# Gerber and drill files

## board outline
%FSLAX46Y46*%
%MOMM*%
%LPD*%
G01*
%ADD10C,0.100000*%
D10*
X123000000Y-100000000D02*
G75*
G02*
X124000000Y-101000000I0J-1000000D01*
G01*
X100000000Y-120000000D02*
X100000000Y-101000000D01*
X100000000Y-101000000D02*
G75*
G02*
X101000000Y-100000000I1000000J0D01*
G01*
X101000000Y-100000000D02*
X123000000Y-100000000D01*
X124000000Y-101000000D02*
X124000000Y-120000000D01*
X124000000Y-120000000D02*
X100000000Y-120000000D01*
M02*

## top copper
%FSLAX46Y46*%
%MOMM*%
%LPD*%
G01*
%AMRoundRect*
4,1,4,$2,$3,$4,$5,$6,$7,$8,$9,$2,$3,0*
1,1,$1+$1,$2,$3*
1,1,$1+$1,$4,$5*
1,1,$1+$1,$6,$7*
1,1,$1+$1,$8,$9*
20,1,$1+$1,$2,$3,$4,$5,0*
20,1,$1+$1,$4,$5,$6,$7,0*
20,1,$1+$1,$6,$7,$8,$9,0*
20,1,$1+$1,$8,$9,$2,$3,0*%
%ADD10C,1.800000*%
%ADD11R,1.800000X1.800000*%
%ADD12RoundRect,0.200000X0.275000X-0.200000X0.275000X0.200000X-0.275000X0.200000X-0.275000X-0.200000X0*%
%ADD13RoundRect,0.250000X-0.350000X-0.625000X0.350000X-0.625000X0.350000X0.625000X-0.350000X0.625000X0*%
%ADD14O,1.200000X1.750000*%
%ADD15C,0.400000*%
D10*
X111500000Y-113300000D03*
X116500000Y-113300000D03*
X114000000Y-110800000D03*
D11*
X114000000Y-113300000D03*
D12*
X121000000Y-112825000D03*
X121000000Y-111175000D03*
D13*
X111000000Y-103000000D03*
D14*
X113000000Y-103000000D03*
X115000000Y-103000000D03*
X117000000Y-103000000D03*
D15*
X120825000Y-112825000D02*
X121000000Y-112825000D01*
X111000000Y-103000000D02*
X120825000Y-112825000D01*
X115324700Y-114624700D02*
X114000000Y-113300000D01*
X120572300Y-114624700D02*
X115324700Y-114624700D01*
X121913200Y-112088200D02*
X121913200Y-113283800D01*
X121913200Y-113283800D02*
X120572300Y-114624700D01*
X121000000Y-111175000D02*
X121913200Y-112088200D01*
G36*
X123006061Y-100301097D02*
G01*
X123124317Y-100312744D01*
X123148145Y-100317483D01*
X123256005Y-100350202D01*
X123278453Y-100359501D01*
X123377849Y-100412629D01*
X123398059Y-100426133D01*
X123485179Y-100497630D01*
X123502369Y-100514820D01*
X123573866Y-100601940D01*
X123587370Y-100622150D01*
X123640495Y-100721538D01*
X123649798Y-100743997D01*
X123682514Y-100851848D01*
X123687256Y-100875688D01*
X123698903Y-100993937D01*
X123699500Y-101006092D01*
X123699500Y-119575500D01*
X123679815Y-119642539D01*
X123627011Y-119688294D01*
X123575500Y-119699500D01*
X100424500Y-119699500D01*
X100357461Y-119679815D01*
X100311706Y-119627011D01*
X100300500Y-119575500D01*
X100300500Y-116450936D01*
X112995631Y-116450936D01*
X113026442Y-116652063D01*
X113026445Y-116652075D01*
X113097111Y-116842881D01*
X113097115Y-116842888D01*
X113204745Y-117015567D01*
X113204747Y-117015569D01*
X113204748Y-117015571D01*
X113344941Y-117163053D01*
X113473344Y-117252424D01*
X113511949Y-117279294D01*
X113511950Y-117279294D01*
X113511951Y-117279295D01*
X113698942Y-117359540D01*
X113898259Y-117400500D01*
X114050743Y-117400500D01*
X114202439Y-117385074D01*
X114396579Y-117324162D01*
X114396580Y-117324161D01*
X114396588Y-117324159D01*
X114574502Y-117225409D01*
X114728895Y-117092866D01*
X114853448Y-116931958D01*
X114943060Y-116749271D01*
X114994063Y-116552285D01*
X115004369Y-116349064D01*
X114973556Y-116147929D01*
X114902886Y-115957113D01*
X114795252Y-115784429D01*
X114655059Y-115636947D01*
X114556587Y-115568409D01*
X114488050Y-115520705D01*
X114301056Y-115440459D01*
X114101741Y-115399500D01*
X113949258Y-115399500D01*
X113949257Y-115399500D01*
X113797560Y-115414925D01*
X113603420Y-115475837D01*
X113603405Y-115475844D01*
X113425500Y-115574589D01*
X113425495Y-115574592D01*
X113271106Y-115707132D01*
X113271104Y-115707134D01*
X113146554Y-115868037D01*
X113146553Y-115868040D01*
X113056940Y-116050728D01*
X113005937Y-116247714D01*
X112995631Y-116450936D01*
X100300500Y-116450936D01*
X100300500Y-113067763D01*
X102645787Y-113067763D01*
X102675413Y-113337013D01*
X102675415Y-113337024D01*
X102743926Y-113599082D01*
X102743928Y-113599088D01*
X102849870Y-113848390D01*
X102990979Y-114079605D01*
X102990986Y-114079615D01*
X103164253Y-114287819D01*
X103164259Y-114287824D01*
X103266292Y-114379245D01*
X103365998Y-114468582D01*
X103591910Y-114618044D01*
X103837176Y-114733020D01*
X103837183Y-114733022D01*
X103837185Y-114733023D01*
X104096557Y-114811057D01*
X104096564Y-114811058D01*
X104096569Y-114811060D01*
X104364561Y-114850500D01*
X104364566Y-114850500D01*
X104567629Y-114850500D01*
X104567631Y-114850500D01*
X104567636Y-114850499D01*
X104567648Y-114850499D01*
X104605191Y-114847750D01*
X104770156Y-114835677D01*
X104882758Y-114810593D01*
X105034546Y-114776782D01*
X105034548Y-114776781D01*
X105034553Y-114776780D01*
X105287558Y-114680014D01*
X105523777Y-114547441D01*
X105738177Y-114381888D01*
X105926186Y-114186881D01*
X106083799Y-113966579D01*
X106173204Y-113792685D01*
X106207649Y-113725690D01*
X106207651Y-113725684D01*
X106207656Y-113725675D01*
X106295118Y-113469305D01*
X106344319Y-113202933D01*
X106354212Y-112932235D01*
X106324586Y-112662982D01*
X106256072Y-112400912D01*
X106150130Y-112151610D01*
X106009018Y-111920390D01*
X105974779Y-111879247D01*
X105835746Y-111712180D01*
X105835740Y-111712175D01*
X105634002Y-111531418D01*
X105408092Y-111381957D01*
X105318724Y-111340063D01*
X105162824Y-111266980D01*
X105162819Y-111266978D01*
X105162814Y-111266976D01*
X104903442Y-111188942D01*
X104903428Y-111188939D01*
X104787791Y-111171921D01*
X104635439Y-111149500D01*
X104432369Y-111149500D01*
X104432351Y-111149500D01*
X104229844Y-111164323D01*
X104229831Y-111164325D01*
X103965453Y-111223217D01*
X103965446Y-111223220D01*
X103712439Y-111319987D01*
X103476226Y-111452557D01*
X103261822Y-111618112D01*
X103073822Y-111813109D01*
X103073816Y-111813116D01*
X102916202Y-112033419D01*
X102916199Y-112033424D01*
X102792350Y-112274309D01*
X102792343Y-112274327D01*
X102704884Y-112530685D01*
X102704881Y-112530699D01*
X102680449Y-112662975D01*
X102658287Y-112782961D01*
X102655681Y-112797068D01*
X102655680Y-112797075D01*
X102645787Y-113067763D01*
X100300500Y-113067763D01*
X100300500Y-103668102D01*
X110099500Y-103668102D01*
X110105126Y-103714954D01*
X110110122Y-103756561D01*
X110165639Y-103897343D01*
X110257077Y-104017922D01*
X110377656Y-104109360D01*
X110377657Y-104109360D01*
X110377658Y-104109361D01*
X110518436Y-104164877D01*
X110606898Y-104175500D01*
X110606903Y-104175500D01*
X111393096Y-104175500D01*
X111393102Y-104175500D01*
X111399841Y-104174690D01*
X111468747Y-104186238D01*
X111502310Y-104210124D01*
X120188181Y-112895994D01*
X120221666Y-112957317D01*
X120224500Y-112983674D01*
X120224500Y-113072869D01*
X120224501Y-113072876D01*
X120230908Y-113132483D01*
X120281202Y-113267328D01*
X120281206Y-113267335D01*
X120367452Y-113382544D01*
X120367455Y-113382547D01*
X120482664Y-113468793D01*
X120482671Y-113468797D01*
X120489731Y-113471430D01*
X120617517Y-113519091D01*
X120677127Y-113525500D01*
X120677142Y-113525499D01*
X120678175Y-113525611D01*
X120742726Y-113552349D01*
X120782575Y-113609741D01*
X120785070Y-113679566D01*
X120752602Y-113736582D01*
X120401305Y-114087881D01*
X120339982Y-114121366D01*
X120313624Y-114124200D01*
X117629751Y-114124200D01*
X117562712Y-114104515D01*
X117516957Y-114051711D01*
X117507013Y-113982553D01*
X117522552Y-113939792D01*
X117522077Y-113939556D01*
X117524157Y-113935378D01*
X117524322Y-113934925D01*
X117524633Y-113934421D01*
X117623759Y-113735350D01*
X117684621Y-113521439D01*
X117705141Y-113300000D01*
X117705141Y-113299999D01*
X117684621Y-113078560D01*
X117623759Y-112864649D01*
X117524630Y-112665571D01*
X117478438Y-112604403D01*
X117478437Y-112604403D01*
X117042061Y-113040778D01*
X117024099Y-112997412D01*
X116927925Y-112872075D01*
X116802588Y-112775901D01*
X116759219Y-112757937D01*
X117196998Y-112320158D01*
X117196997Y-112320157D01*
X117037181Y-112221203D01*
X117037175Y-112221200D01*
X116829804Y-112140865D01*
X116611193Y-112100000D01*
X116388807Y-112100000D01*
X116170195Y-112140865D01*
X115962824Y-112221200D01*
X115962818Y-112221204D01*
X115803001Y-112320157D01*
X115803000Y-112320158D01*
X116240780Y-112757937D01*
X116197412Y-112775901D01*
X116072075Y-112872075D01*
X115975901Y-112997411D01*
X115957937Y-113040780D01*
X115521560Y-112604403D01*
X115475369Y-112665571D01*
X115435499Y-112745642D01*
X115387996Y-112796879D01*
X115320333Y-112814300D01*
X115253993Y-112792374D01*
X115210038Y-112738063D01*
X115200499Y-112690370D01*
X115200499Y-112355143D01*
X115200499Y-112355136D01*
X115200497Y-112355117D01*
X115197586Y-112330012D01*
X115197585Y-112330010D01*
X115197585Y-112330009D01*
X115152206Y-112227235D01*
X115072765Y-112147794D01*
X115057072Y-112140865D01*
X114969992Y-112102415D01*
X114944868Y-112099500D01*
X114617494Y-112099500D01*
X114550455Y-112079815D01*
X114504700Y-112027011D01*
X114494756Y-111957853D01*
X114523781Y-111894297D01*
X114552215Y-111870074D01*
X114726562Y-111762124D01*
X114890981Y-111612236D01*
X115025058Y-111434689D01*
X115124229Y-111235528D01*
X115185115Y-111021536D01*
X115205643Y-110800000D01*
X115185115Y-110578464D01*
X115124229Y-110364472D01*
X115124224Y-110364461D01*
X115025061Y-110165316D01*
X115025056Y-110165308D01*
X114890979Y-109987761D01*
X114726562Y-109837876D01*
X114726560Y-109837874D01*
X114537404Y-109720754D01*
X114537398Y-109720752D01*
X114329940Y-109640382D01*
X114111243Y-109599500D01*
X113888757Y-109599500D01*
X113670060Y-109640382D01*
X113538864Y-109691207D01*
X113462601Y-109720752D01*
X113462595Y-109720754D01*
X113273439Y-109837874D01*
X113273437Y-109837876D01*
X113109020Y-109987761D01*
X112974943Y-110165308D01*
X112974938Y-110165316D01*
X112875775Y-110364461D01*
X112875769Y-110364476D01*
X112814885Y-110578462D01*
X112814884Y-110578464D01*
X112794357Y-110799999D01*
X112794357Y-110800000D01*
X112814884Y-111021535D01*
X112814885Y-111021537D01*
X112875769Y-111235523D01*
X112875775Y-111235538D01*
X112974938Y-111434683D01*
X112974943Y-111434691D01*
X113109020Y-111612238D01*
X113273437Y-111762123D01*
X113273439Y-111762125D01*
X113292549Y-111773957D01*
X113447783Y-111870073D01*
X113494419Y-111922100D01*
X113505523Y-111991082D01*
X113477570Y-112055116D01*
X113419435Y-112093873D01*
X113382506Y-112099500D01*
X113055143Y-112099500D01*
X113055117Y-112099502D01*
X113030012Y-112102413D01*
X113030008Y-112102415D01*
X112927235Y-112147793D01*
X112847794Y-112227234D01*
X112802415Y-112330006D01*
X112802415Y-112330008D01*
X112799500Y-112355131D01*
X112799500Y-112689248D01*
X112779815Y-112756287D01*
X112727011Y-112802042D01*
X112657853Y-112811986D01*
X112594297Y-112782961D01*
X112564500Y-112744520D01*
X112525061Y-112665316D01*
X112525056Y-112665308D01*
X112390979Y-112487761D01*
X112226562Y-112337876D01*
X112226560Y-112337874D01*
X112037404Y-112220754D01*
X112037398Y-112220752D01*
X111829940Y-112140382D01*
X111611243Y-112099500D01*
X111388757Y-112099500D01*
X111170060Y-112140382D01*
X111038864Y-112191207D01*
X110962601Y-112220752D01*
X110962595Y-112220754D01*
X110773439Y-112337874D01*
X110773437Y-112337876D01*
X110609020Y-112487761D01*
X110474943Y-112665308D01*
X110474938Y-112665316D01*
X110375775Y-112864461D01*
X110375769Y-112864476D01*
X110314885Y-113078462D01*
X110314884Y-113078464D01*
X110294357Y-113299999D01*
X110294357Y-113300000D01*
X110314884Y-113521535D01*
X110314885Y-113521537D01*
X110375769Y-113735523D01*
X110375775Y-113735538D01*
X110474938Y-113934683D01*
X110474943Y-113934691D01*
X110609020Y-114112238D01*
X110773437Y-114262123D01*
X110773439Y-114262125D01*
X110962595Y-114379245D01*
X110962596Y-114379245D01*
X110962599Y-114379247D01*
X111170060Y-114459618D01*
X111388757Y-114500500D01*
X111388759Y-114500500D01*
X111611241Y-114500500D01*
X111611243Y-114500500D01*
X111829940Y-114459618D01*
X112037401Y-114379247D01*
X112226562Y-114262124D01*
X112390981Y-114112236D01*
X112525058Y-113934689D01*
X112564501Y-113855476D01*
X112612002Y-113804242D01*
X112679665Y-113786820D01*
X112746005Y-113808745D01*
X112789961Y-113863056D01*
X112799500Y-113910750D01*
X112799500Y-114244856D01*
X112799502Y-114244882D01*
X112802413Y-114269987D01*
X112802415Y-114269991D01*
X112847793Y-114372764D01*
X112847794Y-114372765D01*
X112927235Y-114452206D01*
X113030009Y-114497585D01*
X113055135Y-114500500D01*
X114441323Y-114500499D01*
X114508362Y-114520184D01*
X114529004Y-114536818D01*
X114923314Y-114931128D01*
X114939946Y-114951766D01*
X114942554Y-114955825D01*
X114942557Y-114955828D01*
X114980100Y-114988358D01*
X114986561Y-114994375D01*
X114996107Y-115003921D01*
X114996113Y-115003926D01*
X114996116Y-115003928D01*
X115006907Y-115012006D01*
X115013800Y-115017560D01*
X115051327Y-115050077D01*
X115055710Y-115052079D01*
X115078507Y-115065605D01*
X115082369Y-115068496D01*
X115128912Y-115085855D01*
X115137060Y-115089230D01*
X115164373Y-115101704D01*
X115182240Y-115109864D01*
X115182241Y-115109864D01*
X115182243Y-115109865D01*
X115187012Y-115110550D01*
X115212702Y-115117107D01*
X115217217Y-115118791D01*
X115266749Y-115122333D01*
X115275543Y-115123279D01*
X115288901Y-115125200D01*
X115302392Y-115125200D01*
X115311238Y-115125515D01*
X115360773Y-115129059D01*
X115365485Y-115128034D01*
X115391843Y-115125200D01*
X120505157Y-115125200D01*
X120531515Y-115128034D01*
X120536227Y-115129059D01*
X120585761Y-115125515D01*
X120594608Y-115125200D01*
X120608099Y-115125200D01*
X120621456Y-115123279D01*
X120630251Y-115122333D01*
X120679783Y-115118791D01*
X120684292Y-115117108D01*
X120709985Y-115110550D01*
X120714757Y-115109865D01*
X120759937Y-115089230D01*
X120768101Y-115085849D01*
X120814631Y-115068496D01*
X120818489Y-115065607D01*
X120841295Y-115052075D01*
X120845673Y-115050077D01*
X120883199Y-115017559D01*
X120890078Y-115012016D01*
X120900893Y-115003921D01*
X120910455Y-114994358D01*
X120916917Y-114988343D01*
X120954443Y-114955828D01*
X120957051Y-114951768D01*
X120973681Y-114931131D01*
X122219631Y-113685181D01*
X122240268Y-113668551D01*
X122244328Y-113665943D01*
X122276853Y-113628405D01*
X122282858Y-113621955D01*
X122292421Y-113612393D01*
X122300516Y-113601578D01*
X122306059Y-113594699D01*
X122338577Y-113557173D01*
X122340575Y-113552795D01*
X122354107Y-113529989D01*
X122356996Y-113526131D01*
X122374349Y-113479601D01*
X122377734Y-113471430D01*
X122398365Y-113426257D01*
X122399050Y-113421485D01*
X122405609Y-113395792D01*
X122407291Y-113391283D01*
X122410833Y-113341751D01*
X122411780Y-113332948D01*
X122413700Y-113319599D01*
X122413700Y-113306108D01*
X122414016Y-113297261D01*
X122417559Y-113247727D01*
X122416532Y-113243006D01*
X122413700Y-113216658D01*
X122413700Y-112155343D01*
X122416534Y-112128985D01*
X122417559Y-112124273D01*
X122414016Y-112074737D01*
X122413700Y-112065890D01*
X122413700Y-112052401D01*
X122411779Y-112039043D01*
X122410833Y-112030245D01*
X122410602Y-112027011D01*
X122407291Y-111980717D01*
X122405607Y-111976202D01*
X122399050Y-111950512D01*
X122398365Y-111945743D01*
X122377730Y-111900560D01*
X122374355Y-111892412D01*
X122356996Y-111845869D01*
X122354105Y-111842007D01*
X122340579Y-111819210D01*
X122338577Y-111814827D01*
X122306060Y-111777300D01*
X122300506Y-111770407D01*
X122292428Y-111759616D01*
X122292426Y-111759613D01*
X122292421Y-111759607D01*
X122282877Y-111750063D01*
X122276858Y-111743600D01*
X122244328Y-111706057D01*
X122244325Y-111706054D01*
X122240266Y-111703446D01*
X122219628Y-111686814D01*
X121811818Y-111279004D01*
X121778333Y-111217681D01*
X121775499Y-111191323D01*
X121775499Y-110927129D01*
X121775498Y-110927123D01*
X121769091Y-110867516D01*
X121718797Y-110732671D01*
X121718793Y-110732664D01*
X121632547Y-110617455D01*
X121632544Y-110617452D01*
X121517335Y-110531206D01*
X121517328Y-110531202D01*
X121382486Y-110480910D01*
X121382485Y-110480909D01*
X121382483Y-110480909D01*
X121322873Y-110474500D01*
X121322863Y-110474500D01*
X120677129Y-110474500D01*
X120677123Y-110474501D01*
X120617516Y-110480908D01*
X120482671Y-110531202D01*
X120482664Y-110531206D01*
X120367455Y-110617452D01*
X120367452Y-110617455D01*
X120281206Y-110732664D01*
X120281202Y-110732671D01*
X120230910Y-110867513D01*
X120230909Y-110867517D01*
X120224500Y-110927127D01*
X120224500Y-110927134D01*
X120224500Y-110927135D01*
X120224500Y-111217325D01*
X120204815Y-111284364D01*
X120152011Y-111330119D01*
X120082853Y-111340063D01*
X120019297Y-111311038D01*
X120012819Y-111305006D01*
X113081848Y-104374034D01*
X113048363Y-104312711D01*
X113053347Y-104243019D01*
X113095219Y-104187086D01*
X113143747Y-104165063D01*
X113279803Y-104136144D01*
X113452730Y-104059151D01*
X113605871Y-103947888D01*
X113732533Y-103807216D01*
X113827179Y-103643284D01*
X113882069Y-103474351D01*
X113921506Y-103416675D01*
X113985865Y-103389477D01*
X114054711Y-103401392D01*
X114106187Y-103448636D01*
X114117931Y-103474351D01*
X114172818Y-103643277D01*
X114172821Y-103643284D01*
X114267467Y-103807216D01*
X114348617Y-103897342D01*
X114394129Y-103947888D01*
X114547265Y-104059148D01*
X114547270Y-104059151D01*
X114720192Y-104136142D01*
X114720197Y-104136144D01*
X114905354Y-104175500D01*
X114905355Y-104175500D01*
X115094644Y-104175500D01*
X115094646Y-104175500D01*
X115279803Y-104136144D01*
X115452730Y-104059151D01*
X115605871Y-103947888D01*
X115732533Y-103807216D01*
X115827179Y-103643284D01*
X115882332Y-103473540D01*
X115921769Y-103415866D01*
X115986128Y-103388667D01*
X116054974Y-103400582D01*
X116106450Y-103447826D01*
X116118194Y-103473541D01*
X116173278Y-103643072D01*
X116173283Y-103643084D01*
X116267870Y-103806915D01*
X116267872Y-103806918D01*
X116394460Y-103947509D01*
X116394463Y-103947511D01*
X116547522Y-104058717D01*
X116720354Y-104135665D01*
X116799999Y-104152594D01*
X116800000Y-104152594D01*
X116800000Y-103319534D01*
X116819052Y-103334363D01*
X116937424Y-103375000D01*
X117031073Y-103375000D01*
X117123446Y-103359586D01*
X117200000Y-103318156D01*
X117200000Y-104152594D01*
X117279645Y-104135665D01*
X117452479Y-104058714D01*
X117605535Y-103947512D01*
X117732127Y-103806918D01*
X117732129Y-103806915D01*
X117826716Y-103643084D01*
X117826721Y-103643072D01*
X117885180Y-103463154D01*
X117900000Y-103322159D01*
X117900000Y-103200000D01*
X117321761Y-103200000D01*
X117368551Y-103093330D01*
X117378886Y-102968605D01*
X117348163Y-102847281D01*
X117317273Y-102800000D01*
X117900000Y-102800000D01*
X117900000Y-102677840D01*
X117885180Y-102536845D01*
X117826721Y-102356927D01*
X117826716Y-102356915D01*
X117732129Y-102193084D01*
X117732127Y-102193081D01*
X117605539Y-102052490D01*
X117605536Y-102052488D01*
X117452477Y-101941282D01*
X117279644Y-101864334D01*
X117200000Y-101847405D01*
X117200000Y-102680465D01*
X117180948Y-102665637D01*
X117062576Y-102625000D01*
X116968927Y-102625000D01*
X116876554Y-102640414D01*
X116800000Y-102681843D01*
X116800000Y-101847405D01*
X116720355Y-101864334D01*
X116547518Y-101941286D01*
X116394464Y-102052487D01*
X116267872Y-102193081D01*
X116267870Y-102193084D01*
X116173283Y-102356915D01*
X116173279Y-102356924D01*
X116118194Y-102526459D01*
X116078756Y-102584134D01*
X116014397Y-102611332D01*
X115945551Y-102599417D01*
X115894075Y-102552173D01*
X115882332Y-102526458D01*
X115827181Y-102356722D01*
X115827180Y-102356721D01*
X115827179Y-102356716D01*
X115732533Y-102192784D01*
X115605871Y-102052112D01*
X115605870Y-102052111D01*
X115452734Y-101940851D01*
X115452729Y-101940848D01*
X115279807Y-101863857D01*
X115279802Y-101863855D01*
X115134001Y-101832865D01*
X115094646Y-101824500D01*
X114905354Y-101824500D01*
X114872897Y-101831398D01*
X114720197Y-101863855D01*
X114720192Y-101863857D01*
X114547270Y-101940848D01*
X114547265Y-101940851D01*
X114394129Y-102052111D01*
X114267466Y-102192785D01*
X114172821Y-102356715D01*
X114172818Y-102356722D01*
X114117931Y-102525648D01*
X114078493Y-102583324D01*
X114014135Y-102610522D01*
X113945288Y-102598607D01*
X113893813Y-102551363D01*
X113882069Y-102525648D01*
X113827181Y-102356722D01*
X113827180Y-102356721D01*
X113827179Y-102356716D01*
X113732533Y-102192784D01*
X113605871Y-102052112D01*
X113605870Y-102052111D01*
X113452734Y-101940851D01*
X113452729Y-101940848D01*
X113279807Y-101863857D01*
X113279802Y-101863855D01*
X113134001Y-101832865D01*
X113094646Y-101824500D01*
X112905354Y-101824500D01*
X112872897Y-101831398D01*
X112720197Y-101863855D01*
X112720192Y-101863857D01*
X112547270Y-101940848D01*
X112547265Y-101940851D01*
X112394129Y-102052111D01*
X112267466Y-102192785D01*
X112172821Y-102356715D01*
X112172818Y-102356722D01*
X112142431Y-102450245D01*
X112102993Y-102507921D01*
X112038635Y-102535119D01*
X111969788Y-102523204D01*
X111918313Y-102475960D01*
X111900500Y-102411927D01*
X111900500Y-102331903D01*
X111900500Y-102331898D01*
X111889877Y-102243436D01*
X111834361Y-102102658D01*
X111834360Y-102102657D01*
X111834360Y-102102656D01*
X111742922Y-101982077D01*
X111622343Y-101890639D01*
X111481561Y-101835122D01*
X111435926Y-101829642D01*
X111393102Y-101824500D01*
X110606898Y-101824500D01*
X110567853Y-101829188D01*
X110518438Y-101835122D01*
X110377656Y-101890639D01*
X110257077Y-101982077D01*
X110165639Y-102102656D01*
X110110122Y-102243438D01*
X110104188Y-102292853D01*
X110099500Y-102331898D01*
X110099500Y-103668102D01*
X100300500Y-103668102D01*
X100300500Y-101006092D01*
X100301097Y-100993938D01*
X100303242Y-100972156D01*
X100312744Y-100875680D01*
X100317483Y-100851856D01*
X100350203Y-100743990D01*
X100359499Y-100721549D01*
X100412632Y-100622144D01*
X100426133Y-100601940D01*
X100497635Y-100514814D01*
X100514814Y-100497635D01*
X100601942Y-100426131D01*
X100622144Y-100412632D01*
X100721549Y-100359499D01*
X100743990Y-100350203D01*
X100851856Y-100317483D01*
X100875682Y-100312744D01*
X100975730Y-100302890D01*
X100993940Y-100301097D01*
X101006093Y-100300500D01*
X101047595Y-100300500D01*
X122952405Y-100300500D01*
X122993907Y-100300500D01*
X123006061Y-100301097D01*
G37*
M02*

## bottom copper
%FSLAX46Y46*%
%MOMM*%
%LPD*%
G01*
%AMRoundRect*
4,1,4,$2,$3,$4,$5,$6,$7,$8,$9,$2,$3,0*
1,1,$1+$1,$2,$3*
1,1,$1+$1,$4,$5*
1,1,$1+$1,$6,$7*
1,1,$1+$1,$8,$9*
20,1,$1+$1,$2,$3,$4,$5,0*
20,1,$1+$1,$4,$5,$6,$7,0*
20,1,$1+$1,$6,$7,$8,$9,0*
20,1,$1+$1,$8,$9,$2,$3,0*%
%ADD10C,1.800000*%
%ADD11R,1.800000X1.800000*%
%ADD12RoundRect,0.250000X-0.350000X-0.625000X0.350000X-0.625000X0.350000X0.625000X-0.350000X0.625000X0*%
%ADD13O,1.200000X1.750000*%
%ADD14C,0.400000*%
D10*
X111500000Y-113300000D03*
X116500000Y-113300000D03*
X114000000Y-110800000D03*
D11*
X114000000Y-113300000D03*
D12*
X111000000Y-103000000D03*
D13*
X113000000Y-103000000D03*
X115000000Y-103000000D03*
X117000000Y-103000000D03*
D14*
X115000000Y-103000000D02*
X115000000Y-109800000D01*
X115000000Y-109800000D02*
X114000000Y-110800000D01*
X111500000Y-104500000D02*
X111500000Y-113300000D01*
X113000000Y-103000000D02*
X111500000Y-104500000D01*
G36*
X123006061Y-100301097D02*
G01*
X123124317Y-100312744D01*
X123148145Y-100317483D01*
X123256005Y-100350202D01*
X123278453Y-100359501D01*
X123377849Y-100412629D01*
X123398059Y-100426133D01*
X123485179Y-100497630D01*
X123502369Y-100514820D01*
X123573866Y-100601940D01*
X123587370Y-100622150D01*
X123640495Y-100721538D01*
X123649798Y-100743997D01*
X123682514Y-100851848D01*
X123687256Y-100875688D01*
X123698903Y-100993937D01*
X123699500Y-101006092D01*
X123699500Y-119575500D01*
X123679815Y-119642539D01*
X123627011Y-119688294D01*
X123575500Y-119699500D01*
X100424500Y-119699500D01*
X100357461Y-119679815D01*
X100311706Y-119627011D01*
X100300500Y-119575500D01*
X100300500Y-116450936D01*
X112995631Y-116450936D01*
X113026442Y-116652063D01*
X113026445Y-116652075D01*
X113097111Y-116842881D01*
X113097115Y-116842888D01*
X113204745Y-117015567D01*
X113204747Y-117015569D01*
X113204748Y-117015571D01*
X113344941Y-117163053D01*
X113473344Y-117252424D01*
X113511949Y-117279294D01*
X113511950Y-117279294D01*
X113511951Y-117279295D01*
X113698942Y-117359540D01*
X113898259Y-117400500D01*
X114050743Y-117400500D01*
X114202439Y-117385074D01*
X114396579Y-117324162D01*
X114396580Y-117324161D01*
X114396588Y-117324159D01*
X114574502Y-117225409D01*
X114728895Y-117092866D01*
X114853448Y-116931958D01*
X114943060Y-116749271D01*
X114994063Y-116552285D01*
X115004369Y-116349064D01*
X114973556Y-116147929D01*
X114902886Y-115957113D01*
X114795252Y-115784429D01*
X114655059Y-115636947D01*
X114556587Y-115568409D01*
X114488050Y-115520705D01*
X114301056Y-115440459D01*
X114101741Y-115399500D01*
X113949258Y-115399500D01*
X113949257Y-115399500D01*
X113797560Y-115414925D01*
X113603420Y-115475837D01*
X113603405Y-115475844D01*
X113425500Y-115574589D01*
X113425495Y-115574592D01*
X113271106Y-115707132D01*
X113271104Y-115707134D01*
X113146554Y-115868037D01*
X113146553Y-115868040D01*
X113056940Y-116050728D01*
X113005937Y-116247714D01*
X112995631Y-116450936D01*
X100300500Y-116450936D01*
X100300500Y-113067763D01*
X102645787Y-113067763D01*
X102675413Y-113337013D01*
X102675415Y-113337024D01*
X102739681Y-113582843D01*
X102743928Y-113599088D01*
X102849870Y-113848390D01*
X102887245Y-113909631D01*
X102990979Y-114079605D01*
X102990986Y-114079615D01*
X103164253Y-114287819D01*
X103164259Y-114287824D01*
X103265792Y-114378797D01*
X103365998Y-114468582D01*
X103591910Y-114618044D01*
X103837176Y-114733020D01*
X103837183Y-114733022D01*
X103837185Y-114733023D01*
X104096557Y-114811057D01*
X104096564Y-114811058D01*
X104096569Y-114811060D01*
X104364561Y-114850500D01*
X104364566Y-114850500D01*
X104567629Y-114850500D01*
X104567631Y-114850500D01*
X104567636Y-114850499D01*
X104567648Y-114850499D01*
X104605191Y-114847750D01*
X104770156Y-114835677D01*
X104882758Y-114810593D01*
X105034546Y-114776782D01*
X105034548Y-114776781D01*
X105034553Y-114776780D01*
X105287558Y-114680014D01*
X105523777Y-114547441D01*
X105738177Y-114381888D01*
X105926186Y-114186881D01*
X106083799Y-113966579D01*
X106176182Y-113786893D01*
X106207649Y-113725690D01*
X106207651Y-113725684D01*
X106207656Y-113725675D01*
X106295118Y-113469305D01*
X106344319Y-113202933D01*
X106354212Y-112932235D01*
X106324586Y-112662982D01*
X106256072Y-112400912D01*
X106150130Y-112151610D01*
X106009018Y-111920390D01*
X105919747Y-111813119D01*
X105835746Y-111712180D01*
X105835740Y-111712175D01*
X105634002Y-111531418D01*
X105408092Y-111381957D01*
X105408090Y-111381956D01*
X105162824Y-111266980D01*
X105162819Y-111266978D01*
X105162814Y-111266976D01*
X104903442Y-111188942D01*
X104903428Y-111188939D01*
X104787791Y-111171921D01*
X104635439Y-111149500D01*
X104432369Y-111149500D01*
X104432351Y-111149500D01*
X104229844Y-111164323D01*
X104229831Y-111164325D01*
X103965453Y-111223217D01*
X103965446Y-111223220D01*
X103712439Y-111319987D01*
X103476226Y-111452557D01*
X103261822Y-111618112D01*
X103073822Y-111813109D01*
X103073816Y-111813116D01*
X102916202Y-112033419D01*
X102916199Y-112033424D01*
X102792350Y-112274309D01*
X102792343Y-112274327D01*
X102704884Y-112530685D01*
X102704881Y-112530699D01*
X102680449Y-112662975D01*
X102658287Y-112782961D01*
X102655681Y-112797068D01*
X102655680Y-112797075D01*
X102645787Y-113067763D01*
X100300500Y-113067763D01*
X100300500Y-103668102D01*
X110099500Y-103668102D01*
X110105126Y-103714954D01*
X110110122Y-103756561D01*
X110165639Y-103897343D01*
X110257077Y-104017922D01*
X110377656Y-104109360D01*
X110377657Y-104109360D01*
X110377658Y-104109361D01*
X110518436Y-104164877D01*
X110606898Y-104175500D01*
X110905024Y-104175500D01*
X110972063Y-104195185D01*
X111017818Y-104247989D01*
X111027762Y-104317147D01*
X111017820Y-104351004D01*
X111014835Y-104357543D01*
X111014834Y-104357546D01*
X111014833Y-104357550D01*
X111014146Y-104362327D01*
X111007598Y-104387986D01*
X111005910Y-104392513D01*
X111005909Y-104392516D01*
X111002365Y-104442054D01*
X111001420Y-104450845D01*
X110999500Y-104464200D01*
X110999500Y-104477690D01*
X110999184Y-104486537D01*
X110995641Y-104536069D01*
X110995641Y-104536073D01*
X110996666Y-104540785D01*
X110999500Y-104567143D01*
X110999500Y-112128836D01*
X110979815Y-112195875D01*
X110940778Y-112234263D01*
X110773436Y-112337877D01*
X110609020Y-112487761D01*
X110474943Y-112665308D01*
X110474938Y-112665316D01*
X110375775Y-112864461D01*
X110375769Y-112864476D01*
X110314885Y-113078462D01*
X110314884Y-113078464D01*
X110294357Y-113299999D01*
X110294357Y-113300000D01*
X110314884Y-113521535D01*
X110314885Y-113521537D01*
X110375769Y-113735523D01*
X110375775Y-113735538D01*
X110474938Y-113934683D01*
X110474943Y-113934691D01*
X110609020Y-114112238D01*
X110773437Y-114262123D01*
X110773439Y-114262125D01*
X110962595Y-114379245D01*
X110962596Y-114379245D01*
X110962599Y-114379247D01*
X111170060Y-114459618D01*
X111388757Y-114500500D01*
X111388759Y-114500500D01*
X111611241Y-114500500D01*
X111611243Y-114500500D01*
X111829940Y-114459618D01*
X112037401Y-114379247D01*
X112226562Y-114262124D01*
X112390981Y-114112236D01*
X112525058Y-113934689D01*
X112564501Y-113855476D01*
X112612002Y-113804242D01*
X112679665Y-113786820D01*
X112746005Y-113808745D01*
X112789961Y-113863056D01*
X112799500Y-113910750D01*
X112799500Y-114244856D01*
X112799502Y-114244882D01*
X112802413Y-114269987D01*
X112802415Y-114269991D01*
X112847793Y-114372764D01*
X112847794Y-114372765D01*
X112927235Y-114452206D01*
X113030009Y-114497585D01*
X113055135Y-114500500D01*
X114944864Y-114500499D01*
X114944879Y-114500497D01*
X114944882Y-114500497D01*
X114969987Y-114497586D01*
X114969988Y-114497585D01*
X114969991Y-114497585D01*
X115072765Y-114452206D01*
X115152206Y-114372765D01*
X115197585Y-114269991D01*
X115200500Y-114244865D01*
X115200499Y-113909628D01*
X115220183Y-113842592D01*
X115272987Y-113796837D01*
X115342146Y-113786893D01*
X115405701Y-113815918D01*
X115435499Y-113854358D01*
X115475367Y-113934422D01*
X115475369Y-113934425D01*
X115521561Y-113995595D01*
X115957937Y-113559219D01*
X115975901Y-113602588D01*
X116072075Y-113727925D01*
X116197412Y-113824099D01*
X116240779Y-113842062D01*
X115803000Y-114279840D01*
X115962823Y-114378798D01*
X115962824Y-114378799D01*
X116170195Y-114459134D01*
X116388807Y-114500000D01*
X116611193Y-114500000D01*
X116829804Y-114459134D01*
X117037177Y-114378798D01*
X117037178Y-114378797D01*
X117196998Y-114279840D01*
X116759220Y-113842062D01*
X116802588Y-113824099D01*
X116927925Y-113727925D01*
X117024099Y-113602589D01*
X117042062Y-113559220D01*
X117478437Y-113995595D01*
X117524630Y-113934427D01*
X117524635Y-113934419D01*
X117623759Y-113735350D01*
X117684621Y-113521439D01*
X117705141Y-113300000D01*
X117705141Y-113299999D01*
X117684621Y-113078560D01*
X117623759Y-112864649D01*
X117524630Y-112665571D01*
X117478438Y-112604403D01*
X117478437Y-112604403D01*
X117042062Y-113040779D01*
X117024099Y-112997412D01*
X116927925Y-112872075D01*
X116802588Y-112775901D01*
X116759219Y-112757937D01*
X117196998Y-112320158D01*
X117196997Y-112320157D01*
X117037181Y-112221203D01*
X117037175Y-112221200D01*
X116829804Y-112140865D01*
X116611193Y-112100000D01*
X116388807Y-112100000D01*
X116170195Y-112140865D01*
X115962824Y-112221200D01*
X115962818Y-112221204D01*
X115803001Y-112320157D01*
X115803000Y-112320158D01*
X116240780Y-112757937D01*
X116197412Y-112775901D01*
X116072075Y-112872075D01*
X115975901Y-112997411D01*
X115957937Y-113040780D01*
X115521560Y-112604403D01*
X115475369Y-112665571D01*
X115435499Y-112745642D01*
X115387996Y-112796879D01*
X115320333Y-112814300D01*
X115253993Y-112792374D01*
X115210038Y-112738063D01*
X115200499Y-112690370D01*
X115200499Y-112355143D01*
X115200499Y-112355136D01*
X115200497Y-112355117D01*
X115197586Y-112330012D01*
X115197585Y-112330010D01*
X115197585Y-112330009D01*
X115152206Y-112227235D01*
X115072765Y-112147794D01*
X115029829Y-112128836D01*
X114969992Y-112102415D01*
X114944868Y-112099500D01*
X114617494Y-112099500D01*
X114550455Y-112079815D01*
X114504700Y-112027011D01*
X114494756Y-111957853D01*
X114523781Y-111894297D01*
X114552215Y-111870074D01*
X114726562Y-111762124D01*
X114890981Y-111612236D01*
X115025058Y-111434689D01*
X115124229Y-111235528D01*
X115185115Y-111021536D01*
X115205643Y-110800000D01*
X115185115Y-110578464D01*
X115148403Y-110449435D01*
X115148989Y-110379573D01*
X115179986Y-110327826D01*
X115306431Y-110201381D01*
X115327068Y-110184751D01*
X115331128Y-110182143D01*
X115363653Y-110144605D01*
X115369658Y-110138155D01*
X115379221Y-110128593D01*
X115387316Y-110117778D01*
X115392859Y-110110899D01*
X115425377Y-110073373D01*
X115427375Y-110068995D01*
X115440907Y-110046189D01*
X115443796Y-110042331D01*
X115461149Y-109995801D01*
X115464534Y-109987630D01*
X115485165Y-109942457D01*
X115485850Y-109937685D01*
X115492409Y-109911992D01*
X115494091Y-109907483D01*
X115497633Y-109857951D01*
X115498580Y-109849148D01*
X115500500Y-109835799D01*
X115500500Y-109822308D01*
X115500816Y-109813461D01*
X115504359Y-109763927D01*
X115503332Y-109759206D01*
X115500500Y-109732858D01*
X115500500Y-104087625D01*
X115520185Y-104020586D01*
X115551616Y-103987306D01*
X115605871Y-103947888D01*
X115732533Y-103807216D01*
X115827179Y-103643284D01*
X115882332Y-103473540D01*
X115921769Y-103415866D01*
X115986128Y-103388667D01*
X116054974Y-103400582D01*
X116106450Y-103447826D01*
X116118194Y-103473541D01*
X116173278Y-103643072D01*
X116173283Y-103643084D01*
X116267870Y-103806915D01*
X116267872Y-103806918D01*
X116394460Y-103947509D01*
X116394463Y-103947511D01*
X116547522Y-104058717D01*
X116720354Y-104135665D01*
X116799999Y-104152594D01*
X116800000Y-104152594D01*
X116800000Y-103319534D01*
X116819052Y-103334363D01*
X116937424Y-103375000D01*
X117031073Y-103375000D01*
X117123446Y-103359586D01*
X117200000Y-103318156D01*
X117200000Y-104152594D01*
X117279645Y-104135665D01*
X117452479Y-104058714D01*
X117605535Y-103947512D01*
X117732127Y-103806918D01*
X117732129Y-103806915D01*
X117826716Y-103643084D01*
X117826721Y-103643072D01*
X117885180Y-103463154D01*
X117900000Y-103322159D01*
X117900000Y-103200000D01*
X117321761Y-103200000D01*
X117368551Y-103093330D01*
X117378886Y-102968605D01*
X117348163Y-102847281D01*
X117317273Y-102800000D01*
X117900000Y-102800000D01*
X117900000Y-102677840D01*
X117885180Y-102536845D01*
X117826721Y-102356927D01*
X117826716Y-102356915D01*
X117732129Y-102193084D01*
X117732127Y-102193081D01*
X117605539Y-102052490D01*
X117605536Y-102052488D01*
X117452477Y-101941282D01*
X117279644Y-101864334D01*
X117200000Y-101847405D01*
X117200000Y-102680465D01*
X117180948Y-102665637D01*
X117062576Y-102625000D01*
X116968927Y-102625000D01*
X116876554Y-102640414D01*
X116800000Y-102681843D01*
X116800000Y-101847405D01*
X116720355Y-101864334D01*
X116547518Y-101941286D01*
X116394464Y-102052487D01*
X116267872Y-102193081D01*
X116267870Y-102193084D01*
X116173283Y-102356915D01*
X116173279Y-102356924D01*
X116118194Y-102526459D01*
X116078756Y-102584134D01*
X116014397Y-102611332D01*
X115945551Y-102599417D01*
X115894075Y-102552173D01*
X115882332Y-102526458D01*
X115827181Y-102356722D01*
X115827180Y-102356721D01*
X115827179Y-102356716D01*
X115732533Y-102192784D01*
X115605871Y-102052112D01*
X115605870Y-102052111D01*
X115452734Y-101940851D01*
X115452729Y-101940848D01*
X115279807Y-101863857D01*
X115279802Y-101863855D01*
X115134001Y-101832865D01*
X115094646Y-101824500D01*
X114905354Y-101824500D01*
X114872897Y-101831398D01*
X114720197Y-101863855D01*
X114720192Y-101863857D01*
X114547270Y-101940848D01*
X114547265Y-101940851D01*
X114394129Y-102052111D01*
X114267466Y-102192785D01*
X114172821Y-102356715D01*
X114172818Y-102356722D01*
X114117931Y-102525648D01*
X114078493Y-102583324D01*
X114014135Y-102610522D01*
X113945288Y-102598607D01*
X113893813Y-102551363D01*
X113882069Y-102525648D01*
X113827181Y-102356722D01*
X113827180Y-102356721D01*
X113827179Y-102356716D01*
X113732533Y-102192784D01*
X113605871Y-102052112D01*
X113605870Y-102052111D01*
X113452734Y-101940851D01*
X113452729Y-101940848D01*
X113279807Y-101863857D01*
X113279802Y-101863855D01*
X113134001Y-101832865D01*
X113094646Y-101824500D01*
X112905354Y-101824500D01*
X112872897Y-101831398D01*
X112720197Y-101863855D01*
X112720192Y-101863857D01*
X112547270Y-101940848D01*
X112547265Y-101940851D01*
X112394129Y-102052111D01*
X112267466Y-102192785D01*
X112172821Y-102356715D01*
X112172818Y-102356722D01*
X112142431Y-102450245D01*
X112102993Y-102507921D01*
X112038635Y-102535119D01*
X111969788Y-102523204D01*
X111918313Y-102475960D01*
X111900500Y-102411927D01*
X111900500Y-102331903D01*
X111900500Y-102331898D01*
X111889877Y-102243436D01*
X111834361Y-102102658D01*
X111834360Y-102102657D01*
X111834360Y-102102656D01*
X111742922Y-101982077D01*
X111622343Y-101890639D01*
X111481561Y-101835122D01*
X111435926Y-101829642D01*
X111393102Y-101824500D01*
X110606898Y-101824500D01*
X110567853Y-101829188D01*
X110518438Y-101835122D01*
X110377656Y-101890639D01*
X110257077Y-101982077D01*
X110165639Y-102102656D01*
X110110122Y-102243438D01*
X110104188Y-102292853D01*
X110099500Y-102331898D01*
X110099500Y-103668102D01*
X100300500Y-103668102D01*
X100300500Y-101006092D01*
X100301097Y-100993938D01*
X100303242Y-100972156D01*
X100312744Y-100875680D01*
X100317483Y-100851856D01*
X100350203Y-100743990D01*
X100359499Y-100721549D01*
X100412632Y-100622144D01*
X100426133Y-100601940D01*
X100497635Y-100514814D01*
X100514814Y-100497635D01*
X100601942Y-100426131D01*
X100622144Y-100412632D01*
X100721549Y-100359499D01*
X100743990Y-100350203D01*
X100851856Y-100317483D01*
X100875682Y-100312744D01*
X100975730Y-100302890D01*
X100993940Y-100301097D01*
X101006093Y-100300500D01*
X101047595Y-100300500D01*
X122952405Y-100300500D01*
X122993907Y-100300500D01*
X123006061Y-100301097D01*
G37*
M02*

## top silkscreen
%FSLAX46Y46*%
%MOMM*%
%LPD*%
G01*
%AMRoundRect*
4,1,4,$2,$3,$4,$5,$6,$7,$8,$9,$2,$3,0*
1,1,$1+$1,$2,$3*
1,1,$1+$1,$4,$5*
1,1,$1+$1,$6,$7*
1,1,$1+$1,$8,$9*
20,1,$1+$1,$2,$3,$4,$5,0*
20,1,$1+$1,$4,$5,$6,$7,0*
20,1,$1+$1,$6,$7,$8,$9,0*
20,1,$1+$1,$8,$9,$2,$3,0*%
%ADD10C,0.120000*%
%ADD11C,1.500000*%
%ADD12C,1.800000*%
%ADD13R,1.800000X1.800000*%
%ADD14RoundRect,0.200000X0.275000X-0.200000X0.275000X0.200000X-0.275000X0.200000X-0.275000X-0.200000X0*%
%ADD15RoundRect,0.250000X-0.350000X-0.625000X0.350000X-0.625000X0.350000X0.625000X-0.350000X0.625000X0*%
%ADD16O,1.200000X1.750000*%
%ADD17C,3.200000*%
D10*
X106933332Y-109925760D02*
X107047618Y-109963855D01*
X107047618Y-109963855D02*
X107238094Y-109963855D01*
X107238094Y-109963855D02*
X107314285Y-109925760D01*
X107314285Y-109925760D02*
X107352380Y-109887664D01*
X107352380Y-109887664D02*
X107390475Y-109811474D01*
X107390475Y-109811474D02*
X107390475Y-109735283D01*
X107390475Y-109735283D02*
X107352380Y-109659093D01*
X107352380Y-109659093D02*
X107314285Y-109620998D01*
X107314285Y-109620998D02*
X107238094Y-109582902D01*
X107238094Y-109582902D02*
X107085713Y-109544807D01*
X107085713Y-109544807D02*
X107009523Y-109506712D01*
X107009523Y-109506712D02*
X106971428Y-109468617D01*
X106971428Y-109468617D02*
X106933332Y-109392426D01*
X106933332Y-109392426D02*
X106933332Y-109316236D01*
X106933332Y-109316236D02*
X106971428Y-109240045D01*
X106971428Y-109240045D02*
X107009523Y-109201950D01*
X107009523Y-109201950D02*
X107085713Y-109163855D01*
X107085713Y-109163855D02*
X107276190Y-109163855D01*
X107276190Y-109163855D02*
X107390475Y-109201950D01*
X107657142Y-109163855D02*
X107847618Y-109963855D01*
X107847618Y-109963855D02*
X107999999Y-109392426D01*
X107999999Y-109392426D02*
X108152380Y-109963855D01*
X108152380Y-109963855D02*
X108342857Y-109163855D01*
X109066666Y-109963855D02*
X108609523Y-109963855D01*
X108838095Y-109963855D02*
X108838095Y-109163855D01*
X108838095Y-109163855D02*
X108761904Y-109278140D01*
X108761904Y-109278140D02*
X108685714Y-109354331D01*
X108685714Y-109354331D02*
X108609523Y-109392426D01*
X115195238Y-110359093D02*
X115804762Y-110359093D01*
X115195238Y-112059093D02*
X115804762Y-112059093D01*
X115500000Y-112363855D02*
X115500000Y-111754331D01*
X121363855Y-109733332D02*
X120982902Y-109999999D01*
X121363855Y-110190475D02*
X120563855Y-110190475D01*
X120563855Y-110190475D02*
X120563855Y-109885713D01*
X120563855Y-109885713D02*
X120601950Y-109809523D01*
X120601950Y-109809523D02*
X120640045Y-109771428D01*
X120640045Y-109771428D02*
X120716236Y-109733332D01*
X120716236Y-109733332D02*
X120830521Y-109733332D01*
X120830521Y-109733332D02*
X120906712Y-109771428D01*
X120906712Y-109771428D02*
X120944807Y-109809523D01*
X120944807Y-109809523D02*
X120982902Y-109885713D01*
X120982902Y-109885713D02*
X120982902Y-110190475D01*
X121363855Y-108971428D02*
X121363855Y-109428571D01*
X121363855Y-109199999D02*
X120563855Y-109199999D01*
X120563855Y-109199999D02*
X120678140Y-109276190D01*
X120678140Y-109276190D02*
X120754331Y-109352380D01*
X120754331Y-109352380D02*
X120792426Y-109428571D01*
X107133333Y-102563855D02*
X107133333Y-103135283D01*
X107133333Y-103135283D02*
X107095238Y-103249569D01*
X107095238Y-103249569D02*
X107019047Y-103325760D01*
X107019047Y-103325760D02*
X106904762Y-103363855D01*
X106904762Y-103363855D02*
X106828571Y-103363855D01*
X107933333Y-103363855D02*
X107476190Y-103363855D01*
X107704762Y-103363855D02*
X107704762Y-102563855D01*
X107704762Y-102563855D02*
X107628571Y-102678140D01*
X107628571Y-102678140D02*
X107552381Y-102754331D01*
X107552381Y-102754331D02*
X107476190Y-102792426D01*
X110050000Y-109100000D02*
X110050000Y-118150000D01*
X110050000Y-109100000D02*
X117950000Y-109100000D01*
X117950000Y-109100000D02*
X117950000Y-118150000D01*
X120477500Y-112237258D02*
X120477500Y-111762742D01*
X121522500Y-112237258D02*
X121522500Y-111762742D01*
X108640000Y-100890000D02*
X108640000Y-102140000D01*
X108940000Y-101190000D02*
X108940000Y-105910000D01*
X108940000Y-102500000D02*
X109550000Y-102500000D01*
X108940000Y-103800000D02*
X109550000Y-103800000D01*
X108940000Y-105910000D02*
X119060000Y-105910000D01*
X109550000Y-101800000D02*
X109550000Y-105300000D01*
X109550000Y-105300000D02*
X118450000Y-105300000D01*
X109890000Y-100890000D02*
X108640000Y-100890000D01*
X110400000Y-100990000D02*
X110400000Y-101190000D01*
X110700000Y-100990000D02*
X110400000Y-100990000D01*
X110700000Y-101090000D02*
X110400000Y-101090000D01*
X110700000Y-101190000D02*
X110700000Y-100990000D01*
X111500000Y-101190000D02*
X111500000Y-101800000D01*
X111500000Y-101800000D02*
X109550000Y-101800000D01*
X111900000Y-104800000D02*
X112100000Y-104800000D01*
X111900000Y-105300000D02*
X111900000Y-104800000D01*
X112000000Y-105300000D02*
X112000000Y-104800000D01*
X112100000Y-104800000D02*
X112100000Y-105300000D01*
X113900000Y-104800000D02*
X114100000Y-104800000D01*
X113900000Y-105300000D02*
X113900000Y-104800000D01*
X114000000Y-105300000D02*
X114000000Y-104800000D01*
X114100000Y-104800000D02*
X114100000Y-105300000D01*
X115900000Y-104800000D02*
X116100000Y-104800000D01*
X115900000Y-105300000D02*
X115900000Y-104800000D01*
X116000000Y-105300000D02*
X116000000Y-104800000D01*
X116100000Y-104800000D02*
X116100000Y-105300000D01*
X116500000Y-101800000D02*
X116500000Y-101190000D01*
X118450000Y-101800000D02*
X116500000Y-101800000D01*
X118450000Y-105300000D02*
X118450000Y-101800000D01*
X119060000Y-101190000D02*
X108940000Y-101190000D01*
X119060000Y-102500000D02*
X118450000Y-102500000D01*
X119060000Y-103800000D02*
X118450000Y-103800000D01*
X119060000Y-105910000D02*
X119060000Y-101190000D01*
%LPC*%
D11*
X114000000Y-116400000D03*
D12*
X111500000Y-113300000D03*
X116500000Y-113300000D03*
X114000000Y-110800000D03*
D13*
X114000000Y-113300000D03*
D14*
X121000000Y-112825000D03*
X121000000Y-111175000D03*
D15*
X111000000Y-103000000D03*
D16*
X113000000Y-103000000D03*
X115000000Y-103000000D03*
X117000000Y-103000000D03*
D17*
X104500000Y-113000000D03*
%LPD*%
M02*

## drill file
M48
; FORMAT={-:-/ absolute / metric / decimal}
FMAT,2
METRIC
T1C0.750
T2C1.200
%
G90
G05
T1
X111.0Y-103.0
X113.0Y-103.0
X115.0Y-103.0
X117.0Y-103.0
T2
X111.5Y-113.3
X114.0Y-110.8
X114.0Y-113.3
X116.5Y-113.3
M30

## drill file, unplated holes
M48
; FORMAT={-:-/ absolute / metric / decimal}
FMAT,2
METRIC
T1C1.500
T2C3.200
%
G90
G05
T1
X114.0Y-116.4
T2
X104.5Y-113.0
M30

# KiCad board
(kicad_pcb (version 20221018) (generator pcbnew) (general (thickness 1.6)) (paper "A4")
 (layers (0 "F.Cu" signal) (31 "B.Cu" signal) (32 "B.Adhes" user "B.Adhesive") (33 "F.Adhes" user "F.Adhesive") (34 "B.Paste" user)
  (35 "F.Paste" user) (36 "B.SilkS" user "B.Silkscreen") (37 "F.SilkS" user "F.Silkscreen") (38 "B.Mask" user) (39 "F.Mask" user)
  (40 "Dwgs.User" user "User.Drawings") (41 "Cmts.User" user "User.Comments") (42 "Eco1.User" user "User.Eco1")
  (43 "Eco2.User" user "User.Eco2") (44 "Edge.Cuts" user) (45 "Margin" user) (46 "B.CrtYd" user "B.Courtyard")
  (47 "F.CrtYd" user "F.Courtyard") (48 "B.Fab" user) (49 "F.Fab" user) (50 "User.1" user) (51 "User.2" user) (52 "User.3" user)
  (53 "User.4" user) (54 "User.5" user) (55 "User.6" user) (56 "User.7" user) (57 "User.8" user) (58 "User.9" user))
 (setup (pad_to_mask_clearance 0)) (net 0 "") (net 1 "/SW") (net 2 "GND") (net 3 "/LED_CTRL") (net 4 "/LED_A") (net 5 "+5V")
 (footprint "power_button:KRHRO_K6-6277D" (layer "F.Cu") (at 114 113.3)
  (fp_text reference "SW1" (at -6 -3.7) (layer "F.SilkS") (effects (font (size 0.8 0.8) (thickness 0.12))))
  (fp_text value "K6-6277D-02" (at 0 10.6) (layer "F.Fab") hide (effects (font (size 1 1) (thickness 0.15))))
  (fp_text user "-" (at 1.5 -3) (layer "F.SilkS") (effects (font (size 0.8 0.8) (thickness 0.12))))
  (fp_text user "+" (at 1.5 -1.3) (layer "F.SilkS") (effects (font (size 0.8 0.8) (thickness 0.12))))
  (fp_line (start -3.95 -4.2) (end -3.95 4.85) (stroke (width 0.12) (type solid)) (layer "F.SilkS"))
  (fp_line (start -3.95 -4.2) (end 3.95 -4.2) (stroke (width 0.12) (type solid)) (layer "F.SilkS"))
  (fp_line (start 3.95 -4.2) (end 3.95 4.85) (stroke (width 0.12) (type solid)) (layer "F.SilkS"))
  (pad "" np_thru_hole circle (at 0 3.1) (size 1.5 1.5) (drill 1.5) (layers "*.Cu" "*.Mask"))
  (pad "1" thru_hole circle (at -2.5 0) (size 1.8 1.8) (drill 1.2) (layers "*.Cu" "*.Mask") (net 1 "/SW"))
  (pad "2" thru_hole circle (at 2.5 0) (size 1.8 1.8) (drill 1.2) (layers "*.Cu" "*.Mask") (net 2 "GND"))
  (pad "3" thru_hole circle (at 0 -2.5) (size 1.8 1.8) (drill 1.2) (layers "*.Cu" "*.Mask") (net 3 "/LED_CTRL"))
  (pad "4" thru_hole rect (at 0 0) (size 1.8 1.8) (drill 1.2) (layers "*.Cu" "*.Mask") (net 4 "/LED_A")))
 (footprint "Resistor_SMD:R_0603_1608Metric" (layer "F.Cu") (at 121 112 90)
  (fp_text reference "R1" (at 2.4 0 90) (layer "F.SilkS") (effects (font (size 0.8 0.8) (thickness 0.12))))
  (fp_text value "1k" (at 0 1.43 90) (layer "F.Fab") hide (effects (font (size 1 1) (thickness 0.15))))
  (fp_line (start -0.237258 -0.5225) (end 0.237258 -0.5225) (stroke (width 0.12) (type solid)) (layer "F.SilkS"))
  (fp_line (start -0.237258 0.5225) (end 0.237258 0.5225) (stroke (width 0.12) (type solid)) (layer "F.SilkS"))
  (pad "1" smd roundrect (at -0.825 0 90) (size 0.8 0.95) (layers "F.Cu" "F.Paste" "F.Mask") (roundrect_rratio 0.25) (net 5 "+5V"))
  (pad "2" smd roundrect (at 0.825 0 90) (size 0.8 0.95) (layers "F.Cu" "F.Paste" "F.Mask") (roundrect_rratio 0.25) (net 4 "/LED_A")))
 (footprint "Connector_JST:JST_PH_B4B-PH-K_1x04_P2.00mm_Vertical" (layer "F.Cu") (at 111 103)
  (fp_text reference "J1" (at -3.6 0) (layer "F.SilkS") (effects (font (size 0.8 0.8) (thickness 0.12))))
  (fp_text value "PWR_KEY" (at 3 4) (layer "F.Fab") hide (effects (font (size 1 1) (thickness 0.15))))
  (fp_line (start -2.36 -2.11) (end -2.36 -0.86) (stroke (width 0.12) (type solid)) (layer "F.SilkS"))
  (fp_line (start -2.06 -1.81) (end -2.06 2.91) (stroke (width 0.12) (type solid)) (layer "F.SilkS"))
  (fp_line (start -2.06 -0.5) (end -1.45 -0.5) (stroke (width 0.12) (type solid)) (layer "F.SilkS"))
  (fp_line (start -2.06 0.8) (end -1.45 0.8) (stroke (width 0.12) (type solid)) (layer "F.SilkS"))
  (fp_line (start -2.06 2.91) (end 8.06 2.91) (stroke (width 0.12) (type solid)) (layer "F.SilkS"))
  (fp_line (start -1.45 -1.2) (end -1.45 2.3) (stroke (width 0.12) (type solid)) (layer "F.SilkS"))
  (fp_line (start -1.45 2.3) (end 7.45 2.3) (stroke (width 0.12) (type solid)) (layer "F.SilkS"))
  (fp_line (start -1.11 -2.11) (end -2.36 -2.11) (stroke (width 0.12) (type solid)) (layer "F.SilkS"))
  (fp_line (start -0.6 -2.01) (end -0.6 -1.81) (stroke (width 0.12) (type solid)) (layer "F.SilkS"))
  (fp_line (start -0.3 -2.01) (end -0.6 -2.01) (stroke (width 0.12) (type solid)) (layer "F.SilkS"))
  (fp_line (start -0.3 -1.91) (end -0.6 -1.91) (stroke (width 0.12) (type solid)) (layer "F.SilkS"))
  (fp_line (start -0.3 -1.81) (end -0.3 -2.01) (stroke (width 0.12) (type solid)) (layer "F.SilkS"))
  (fp_line (start 0.5 -1.81) (end 0.5 -1.2) (stroke (width 0.12) (type solid)) (layer "F.SilkS"))
  (fp_line (start 0.5 -1.2) (end -1.45 -1.2) (stroke (width 0.12) (type solid)) (layer "F.SilkS"))
  (fp_line (start 0.9 1.8) (end 1.1 1.8) (stroke (width 0.12) (type solid)) (layer "F.SilkS"))
  (fp_line (start 0.9 2.3) (end 0.9 1.8) (stroke (width 0.12) (type solid)) (layer "F.SilkS"))
  (fp_line (start 1 2.3) (end 1 1.8) (stroke (width 0.12) (type solid)) (layer "F.SilkS"))
  (fp_line (start 1.1 1.8) (end 1.1 2.3) (stroke (width 0.12) (type solid)) (layer "F.SilkS"))
  (fp_line (start 2.9 1.8) (end 3.1 1.8) (stroke (width 0.12) (type solid)) (layer "F.SilkS"))
  (fp_line (start 2.9 2.3) (end 2.9 1.8) (stroke (width 0.12) (type solid)) (layer "F.SilkS"))
  (fp_line (start 3 2.3) (end 3 1.8) (stroke (width 0.12) (type solid)) (layer "F.SilkS"))
  (fp_line (start 3.1 1.8) (end 3.1 2.3) (stroke (width 0.12) (type solid)) (layer "F.SilkS"))
  (fp_line (start 4.9 1.8) (end 5.1 1.8) (stroke (width 0.12) (type solid)) (layer "F.SilkS"))
  (fp_line (start 4.9 2.3) (end 4.9 1.8) (stroke (width 0.12) (type solid)) (layer "F.SilkS"))
  (fp_line (start 5 2.3) (end 5 1.8) (stroke (width 0.12) (type solid)) (layer "F.SilkS"))
  (fp_line (start 5.1 1.8) (end 5.1 2.3) (stroke (width 0.12) (type solid)) (layer "F.SilkS"))
  (fp_line (start 5.5 -1.2) (end 5.5 -1.81) (stroke (width 0.12) (type solid)) (layer "F.SilkS"))
  (fp_line (start 7.45 -1.2) (end 5.5 -1.2) (stroke (width 0.12) (type solid)) (layer "F.SilkS"))
  (fp_line (start 7.45 2.3) (end 7.45 -1.2) (stroke (width 0.12) (type solid)) (layer "F.SilkS"))
  (fp_line (start 8.06 -1.81) (end -2.06 -1.81) (stroke (width 0.12) (type solid)) (layer "F.SilkS"))
  (fp_line (start 8.06 -0.5) (end 7.45 -0.5) (stroke (width 0.12) (type solid)) (layer "F.SilkS"))
  (fp_line (start 8.06 0.8) (end 7.45 0.8) (stroke (width 0.12) (type solid)) (layer "F.SilkS"))
  (fp_line (start 8.06 2.91) (end 8.06 -1.81) (stroke (width 0.12) (type solid)) (layer "F.SilkS"))
  (pad "1" thru_hole roundrect (at 0 0) (size 1.2 1.75) (drill 0.75) (layers "*.Cu" "*.Mask") (roundrect_rratio 0.208333) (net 5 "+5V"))
  (pad "2" thru_hole oval (at 2 0) (size 1.2 1.75) (drill 0.75) (layers "*.Cu" "*.Mask") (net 1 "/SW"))
  (pad "3" thru_hole oval (at 4 0) (size 1.2 1.75) (drill 0.75) (layers "*.Cu" "*.Mask") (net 3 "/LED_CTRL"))
  (pad "4" thru_hole oval (at 6 0) (size 1.2 1.75) (drill 0.75) (layers "*.Cu" "*.Mask") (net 2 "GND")))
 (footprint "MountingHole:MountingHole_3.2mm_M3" (layer "F.Cu") (at 104.5 113)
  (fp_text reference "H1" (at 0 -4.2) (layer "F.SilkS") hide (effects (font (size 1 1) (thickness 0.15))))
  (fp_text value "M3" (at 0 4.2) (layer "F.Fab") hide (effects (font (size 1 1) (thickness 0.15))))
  (pad "" np_thru_hole circle (at 0 0) (size 3.2 3.2) (drill 3.2) (layers "*.Cu" "*.Mask")))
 (gr_arc (start 123 100) (mid 123.707107 100.292893) (end 124 101) (stroke (width 0.1) (type default)) (layer "Edge.Cuts"))
 (gr_line (start 100 120) (end 100 101) (stroke (width 0.1) (type default)) (layer "Edge.Cuts"))
 (gr_arc (start 100 101) (mid 100.292893 100.292893) (end 101 100) (stroke (width 0.1) (type default)) (layer "Edge.Cuts"))
 (gr_line (start 101 100) (end 123 100) (stroke (width 0.1) (type default)) (layer "Edge.Cuts"))
 (gr_line (start 124 101) (end 124 120) (stroke (width 0.1) (type default)) (layer "Edge.Cuts"))
 (gr_line (start 124 120) (end 100 120) (stroke (width 0.1) (type default)) (layer "Edge.Cuts"))
 (segment (start 120.825 112.825) (end 121 112.825) (width 0.4) (layer "F.Cu") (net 5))
 (segment (start 111 103) (end 120.825 112.825) (width 0.4) (layer "F.Cu") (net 5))
 (segment (start 115.3247 114.6247) (end 114 113.3) (width 0.4) (layer "F.Cu") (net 4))
 (segment (start 120.5723 114.6247) (end 115.3247 114.6247) (width 0.4) (layer "F.Cu") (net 4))
 (segment (start 121.9132 112.0882) (end 121.9132 113.2838) (width 0.4) (layer "F.Cu") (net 4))
 (segment (start 121.9132 113.2838) (end 120.5723 114.6247) (width 0.4) (layer "F.Cu") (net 4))
 (segment (start 121 111.175) (end 121.9132 112.0882) (width 0.4) (layer "F.Cu") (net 4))
 (segment (start 115 103) (end 115 109.8) (width 0.4) (layer "B.Cu") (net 3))
 (segment (start 115 109.8) (end 114 110.8) (width 0.4) (layer "B.Cu") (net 3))
 (segment (start 111.5 104.5) (end 111.5 113.3) (width 0.4) (layer "B.Cu") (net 1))
 (segment (start 113 103) (end 111.5 104.5) (width 0.4) (layer "B.Cu") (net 1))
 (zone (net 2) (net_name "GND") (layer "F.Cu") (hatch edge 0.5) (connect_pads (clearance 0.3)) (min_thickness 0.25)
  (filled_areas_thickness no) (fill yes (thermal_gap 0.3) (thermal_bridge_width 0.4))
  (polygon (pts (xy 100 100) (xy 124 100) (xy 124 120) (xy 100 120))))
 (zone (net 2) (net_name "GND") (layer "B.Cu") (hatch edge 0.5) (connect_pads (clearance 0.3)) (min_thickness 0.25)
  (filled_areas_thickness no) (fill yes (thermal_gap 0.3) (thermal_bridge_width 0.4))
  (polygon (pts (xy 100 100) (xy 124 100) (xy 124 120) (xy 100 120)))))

